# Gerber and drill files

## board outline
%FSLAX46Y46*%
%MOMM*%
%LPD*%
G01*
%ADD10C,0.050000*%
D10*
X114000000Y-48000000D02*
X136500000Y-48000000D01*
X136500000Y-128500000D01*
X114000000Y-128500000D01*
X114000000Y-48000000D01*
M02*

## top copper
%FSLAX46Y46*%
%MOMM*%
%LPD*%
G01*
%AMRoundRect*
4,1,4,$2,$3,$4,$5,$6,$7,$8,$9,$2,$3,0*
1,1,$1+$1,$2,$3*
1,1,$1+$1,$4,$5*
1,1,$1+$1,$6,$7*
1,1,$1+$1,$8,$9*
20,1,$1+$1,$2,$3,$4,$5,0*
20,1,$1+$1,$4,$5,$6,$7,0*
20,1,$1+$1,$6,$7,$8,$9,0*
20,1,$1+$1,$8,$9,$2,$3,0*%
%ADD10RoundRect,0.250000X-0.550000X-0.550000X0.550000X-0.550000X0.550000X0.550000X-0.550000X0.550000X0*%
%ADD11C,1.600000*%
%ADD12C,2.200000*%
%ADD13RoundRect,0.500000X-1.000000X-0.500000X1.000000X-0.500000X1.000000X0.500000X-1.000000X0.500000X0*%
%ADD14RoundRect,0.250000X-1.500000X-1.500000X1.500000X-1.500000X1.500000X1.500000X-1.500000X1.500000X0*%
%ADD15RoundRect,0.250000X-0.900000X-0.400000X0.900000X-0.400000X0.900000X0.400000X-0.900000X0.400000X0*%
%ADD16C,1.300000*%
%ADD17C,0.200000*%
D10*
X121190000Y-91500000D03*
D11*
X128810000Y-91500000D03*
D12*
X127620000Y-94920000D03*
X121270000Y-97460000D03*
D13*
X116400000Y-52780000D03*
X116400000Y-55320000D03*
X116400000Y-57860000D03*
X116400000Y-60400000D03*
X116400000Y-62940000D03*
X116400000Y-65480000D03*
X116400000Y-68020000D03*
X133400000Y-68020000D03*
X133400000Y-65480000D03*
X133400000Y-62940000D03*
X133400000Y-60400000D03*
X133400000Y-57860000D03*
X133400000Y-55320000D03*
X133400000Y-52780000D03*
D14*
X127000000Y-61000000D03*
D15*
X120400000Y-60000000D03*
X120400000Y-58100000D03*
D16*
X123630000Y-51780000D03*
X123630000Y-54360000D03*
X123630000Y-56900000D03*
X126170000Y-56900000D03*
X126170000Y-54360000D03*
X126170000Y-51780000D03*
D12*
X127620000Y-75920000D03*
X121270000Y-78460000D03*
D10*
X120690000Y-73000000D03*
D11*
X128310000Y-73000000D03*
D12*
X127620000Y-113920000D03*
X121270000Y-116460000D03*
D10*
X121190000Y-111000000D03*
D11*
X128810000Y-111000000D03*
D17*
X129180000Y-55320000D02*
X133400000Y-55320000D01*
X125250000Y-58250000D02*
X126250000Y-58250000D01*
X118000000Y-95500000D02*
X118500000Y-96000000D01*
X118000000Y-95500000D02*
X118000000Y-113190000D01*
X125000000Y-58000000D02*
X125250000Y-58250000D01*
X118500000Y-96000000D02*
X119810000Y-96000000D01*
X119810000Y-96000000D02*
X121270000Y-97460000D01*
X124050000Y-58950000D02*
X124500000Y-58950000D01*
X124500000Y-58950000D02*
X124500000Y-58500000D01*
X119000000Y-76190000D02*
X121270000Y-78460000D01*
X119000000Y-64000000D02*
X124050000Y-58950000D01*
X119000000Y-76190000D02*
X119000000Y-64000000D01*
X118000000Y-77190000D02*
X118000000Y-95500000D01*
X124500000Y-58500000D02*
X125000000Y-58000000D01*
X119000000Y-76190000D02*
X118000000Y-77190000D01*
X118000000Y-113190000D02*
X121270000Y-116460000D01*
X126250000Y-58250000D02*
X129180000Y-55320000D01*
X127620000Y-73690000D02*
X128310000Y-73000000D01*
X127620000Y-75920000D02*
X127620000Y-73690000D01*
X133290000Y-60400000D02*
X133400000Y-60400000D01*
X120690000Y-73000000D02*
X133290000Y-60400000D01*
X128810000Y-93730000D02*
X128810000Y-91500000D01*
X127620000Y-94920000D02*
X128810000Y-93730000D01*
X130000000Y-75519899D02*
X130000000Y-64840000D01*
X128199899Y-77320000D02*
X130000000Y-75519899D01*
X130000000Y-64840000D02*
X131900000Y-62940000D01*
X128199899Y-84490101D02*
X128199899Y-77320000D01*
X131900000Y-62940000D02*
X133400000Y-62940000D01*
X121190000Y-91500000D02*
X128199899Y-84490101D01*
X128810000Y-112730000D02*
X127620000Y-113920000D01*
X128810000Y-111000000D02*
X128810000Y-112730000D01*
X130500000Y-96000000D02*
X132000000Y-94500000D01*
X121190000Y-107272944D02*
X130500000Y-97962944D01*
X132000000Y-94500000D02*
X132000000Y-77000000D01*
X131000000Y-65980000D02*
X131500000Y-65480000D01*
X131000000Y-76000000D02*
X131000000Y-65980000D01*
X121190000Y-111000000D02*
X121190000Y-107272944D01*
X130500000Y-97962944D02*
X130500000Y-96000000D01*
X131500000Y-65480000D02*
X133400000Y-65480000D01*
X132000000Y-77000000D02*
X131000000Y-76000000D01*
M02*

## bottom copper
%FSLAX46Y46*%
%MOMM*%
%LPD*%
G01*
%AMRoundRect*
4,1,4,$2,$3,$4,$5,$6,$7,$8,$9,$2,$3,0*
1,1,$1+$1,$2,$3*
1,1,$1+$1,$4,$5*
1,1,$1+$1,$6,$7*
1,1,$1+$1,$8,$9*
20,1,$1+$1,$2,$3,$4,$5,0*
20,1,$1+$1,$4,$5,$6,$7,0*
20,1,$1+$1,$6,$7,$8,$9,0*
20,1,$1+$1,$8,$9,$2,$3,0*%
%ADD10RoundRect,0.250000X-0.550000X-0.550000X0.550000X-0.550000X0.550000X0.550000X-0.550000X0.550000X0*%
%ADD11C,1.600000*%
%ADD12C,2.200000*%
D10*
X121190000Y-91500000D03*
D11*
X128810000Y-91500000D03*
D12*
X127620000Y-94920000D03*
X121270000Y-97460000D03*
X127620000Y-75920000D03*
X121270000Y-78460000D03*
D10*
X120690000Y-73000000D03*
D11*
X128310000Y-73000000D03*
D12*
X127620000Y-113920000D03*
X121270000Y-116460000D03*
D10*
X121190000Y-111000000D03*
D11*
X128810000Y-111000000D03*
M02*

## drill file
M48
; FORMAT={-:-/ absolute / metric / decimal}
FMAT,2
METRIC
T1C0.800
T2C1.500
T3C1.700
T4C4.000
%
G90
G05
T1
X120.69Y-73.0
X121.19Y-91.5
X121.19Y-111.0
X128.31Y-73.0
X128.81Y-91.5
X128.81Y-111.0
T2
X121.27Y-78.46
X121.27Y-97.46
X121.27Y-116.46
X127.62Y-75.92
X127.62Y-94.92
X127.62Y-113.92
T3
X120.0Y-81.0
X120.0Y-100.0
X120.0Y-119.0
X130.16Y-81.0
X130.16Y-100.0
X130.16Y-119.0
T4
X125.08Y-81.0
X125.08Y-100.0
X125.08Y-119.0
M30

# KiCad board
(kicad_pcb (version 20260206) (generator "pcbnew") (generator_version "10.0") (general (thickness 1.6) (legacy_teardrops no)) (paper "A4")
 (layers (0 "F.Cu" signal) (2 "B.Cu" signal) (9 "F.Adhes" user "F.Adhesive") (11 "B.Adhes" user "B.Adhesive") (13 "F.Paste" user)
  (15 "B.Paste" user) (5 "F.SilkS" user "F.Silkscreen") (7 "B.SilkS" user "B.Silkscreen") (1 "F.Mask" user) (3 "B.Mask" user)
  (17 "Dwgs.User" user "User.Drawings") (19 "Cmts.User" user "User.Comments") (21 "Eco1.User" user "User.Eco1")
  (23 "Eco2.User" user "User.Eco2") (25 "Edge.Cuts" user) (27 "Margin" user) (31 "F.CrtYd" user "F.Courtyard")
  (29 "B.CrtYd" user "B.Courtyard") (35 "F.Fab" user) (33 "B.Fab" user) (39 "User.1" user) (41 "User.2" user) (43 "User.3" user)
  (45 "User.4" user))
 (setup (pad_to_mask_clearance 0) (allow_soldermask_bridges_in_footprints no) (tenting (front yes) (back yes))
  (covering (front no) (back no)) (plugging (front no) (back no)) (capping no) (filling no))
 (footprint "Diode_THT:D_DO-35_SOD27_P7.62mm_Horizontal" (layer "F.Cu") (at 121.19 91.5)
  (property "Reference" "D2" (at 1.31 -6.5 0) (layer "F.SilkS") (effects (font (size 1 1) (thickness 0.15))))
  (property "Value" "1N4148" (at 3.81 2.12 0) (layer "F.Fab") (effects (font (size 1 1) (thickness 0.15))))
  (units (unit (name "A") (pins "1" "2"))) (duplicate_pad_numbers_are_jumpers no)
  (pad "1" thru_hole roundrect (at 0 0) (size 1.6 1.6) (drill 0.8) (layers "*.Cu" "*.Mask") (remove_unused_layers no)
   (roundrect_rratio 0.15625) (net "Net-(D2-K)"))
  (pad "2" thru_hole circle (at 7.62 0) (size 1.6 1.6) (drill 0.8) (layers "*.Cu" "*.Mask") (remove_unused_layers no) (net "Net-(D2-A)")))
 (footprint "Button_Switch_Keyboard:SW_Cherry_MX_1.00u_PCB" (layer "F.Cu") (at 127.62 94.92)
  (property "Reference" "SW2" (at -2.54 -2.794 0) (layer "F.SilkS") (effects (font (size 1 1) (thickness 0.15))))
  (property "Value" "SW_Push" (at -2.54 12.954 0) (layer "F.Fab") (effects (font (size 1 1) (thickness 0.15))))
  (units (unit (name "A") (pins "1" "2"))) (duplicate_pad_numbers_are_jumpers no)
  (pad "" np_thru_hole circle (at -7.62 5.08) (size 1.7 1.7) (drill 1.7) (layers "*.Cu" "*.Mask"))
  (pad "" np_thru_hole circle (at -2.54 5.08) (size 4 4) (drill 4) (layers "*.Cu" "*.Mask"))
  (pad "" np_thru_hole circle (at 2.54 5.08) (size 1.7 1.7) (drill 1.7) (layers "*.Cu" "*.Mask"))
  (pad "1" thru_hole circle (at 0 0) (size 2.2 2.2) (drill 1.5) (layers "*.Cu" "*.Mask") (remove_unused_layers no) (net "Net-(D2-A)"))
  (pad "2" thru_hole circle (at -6.35 2.54) (size 2.2 2.2) (drill 1.5) (layers "*.Cu" "*.Mask") (remove_unused_layers no) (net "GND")))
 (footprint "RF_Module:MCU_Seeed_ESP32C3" (layer "F.Cu") (at 124.9 60.4)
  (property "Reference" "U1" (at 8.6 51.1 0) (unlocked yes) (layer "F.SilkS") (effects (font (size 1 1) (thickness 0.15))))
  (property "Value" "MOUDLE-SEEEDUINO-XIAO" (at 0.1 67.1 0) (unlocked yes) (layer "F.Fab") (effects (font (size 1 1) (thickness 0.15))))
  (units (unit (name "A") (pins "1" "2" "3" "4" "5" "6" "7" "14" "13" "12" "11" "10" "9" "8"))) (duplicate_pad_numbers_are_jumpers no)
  (pad "" smd roundrect (at 1.1 -0.4) (size 1.5 1.5) (layers "F.Paste") (roundrect_rratio 0.1666666667))
  (pad "" smd roundrect (at 1.1 1.6) (size 1.5 1.5) (layers "F.Paste") (roundrect_rratio 0.1666666667))
  (pad "" smd roundrect (at 3.1 -0.4) (size 1.5 1.5) (layers "F.Paste") (roundrect_rratio 0.1666666667))
  (pad "" smd roundrect (at 3.1 1.6) (size 1.5 1.5) (layers "F.Paste") (roundrect_rratio 0.1666666667))
  (pad "1" smd roundrect (at -8.5 -7.62) (size 3 2) (layers "F.Cu" "F.Mask" "F.Paste") (roundrect_rratio 0.25)
   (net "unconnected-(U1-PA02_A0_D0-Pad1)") (thermal_bridge_angle 45))
  (pad "2" smd roundrect (at -8.5 -5.08) (size 3 2) (layers "F.Cu" "F.Mask" "F.Paste") (roundrect_rratio 0.25)
   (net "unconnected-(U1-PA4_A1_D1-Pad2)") (thermal_bridge_angle 45))
  (pad "3" smd roundrect (at -8.5 -2.54) (size 3 2) (layers "F.Cu" "F.Mask" "F.Paste") (roundrect_rratio 0.25)
   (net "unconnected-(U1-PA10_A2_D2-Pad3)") (thermal_bridge_angle 45))
  (pad "4" smd roundrect (at -8.5 0) (size 3 2) (layers "F.Cu" "F.Mask" "F.Paste") (roundrect_rratio 0.25)
   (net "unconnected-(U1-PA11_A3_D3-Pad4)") (thermal_bridge_angle 45))
  (pad "5" smd roundrect (at -8.5 2.54) (size 3 2) (layers "F.Cu" "F.Mask" "F.Paste") (roundrect_rratio 0.25)
   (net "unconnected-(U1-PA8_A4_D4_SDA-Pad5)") (thermal_bridge_angle 45))
  (pad "6" smd roundrect (at -8.5 5.08) (size 3 2) (layers "F.Cu" "F.Mask" "F.Paste") (roundrect_rratio 0.25)
   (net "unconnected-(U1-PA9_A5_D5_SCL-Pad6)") (thermal_bridge_angle 45))
  (pad "7" smd roundrect (at -8.5 7.62) (size 3 2) (layers "F.Cu" "F.Mask" "F.Paste") (roundrect_rratio 0.25)
   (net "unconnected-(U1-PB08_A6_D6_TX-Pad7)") (thermal_bridge_angle 45))
  (pad "8" smd roundrect (at 8.5 7.62) (size 3 2) (layers "F.Cu" "F.Mask" "F.Paste") (roundrect_rratio 0.25)
   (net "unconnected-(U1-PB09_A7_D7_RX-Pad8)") (thermal_bridge_angle 45))
  (pad "9" smd roundrect (at 8.5 5.08) (size 3 2) (layers "F.Cu" "F.Mask" "F.Paste") (roundrect_rratio 0.25) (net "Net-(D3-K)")
   (thermal_bridge_angle 45))
  (pad "10" smd roundrect (at 8.5 2.54) (size 3 2) (layers "F.Cu" "F.Mask" "F.Paste") (roundrect_rratio 0.25) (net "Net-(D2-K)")
   (thermal_bridge_angle 45))
  (pad "11" smd roundrect (at 8.5 0) (size 3 2) (layers "F.Cu" "F.Mask" "F.Paste") (roundrect_rratio 0.25) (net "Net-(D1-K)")
   (thermal_bridge_angle 45))
  (pad "12" smd roundrect (at 8.5 -2.54) (size 3 2) (layers "F.Cu" "F.Mask" "F.Paste") (roundrect_rratio 0.25)
   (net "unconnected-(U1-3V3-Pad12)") (thermal_bridge_angle 45))
  (pad "13" smd roundrect (at 8.5 -5.08) (size 3 2) (layers "F.Cu" "F.Mask" "F.Paste") (roundrect_rratio 0.25) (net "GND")
   (thermal_bridge_angle 45))
  (pad "14" smd roundrect (at 8.5 -7.62) (size 3 2) (layers "F.Cu" "F.Mask" "F.Paste") (roundrect_rratio 0.25)
   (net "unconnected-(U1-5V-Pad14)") (thermal_bridge_angle 45))
  (pad "15" smd roundrect (at 2.1 0.6) (size 3.5 3.5) (layers "F.Cu" "F.Mask") (roundrect_rratio 0.07142857143))
  (pad "16" smd roundrect (at -4.5 -0.4) (size 2.3 1.3) (layers "F.Cu" "F.Mask" "F.Paste") (roundrect_rratio 0.1923076923))
  (pad "17" smd roundrect (at -4.5 -2.3) (size 2.3 1.3) (layers "F.Cu" "F.Mask" "F.Paste") (roundrect_rratio 0.1923076923))
  (pad "18" smd circle (at -1.27 -8.62) (size 1.3 1.3) (layers "F.Cu" "F.Mask" "F.Paste"))
  (pad "19" smd circle (at -1.27 -6.04) (size 1.3 1.3) (layers "F.Cu" "F.Mask" "F.Paste"))
  (pad "20" smd circle (at -1.27 -3.5) (size 1.3 1.3) (layers "F.Cu" "F.Mask" "F.Paste"))
  (pad "21" smd circle (at 1.27 -3.5) (size 1.3 1.3) (layers "F.Cu" "F.Mask" "F.Paste"))
  (pad "22" smd circle (at 1.27 -6.04) (size 1.3 1.3) (layers "F.Cu" "F.Mask" "F.Paste"))
  (pad "23" smd circle (at 1.27 -8.62) (size 1.3 1.3) (layers "F.Cu" "F.Mask" "F.Paste")))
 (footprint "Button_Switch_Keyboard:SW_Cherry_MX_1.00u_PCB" (layer "F.Cu") (at 127.62 75.92)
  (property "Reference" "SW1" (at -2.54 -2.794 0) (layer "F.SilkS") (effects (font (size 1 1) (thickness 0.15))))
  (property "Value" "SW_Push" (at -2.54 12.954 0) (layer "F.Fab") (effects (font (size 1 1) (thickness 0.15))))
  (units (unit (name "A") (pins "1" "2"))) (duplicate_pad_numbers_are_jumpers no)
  (pad "" np_thru_hole circle (at -7.62 5.08) (size 1.7 1.7) (drill 1.7) (layers "*.Cu" "*.Mask"))
  (pad "" np_thru_hole circle (at -2.54 5.08) (size 4 4) (drill 4) (layers "*.Cu" "*.Mask"))
  (pad "" np_thru_hole circle (at 2.54 5.08) (size 1.7 1.7) (drill 1.7) (layers "*.Cu" "*.Mask"))
  (pad "1" thru_hole circle (at 0 0) (size 2.2 2.2) (drill 1.5) (layers "*.Cu" "*.Mask") (remove_unused_layers no) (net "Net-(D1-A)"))
  (pad "2" thru_hole circle (at -6.35 2.54) (size 2.2 2.2) (drill 1.5) (layers "*.Cu" "*.Mask") (remove_unused_layers no) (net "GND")))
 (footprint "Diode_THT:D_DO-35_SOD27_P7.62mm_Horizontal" (layer "F.Cu") (at 120.69 73)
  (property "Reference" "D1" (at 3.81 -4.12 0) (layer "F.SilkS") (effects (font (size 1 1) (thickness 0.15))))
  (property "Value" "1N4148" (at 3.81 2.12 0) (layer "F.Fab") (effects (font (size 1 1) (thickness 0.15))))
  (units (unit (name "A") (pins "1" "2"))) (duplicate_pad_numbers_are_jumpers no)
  (pad "1" thru_hole roundrect (at 0 0) (size 1.6 1.6) (drill 0.8) (layers "*.Cu" "*.Mask") (remove_unused_layers no)
   (roundrect_rratio 0.15625) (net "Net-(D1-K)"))
  (pad "2" thru_hole circle (at 7.62 0) (size 1.6 1.6) (drill 0.8) (layers "*.Cu" "*.Mask") (remove_unused_layers no) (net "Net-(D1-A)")))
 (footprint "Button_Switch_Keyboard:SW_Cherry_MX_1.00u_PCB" (layer "F.Cu") (at 127.62 113.92)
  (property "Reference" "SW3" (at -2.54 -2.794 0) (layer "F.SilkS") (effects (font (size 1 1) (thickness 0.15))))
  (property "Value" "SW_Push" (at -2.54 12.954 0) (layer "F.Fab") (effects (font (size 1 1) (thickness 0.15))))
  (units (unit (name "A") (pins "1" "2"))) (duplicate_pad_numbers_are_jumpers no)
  (pad "" np_thru_hole circle (at -7.62 5.08) (size 1.7 1.7) (drill 1.7) (layers "*.Cu" "*.Mask"))
  (pad "" np_thru_hole circle (at -2.54 5.08) (size 4 4) (drill 4) (layers "*.Cu" "*.Mask"))
  (pad "" np_thru_hole circle (at 2.54 5.08) (size 1.7 1.7) (drill 1.7) (layers "*.Cu" "*.Mask"))
  (pad "1" thru_hole circle (at 0 0) (size 2.2 2.2) (drill 1.5) (layers "*.Cu" "*.Mask") (remove_unused_layers no) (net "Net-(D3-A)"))
  (pad "2" thru_hole circle (at -6.35 2.54) (size 2.2 2.2) (drill 1.5) (layers "*.Cu" "*.Mask") (remove_unused_layers no) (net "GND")))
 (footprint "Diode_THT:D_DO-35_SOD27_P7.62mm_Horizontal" (layer "F.Cu") (at 121.19 111)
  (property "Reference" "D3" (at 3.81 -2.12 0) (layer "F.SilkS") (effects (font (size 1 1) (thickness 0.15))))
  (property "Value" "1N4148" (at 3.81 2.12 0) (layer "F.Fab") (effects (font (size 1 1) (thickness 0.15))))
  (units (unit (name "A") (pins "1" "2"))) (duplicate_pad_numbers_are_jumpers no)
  (pad "1" thru_hole roundrect (at 0 0) (size 1.6 1.6) (drill 0.8) (layers "*.Cu" "*.Mask") (remove_unused_layers no)
   (roundrect_rratio 0.15625) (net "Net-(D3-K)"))
  (pad "2" thru_hole circle (at 7.62 0) (size 1.6 1.6) (drill 0.8) (layers "*.Cu" "*.Mask") (remove_unused_layers no) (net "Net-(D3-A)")))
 (gr_rect (start 114 48) (end 136.5 128.5) (stroke (width 0.05) (type default)) (fill no) (layer "Edge.Cuts"))
 (segment (start 129.18 55.32) (end 133.4 55.32) (width 0.2) (layer "F.Cu") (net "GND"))
 (segment (start 125.25 58.25) (end 126.25 58.25) (width 0.2) (layer "F.Cu") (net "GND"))
 (segment (start 118 95.5) (end 118.5 96) (width 0.2) (layer "F.Cu") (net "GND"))
 (segment (start 118 95.5) (end 118 113.19) (width 0.2) (layer "F.Cu") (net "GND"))
 (segment (start 125 58) (end 125.25 58.25) (width 0.2) (layer "F.Cu") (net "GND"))
 (segment (start 118.5 96) (end 119.81 96) (width 0.2) (layer "F.Cu") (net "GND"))
 (segment (start 119.81 96) (end 121.27 97.46) (width 0.2) (layer "F.Cu") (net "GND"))
 (segment (start 124.05 58.95) (end 124.5 58.95) (width 0.2) (layer "F.Cu") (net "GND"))
 (segment (start 124.5 58.95) (end 124.5 58.5) (width 0.2) (layer "F.Cu") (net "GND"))
 (segment (start 119 76.19) (end 121.27 78.46) (width 0.2) (layer "F.Cu") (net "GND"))
 (segment (start 119 64) (end 124.05 58.95) (width 0.2) (layer "F.Cu") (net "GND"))
 (segment (start 119 76.19) (end 119 64) (width 0.2) (layer "F.Cu") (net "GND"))
 (segment (start 118 77.19) (end 118 95.5) (width 0.2) (layer "F.Cu") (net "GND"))
 (segment (start 124.5 58.5) (end 125 58) (width 0.2) (layer "F.Cu") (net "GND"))
 (segment (start 119 76.19) (end 118 77.19) (width 0.2) (layer "F.Cu") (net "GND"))
 (segment (start 118 113.19) (end 121.27 116.46) (width 0.2) (layer "F.Cu") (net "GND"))
 (segment (start 126.25 58.25) (end 129.18 55.32) (width 0.2) (layer "F.Cu") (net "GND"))
 (segment (start 127.62 73.69) (end 128.31 73) (width 0.2) (layer "F.Cu") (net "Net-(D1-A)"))
 (segment (start 127.62 75.92) (end 127.62 73.69) (width 0.2) (layer "F.Cu") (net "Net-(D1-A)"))
 (segment (start 133.29 60.4) (end 133.4 60.4) (width 0.2) (layer "F.Cu") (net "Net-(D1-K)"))
 (segment (start 120.69 73) (end 133.29 60.4) (width 0.2) (layer "F.Cu") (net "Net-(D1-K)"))
 (segment (start 128.81 93.73) (end 128.81 91.5) (width 0.2) (layer "F.Cu") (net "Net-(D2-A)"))
 (segment (start 127.62 94.92) (end 128.81 93.73) (width 0.2) (layer "F.Cu") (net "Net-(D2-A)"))
 (segment (start 130 75.519899) (end 130 64.84) (width 0.2) (layer "F.Cu") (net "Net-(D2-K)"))
 (segment (start 128.199899 77.32) (end 130 75.519899) (width 0.2) (layer "F.Cu") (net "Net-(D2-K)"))
 (segment (start 130 64.84) (end 131.9 62.94) (width 0.2) (layer "F.Cu") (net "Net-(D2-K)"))
 (segment (start 128.199899 84.490101) (end 128.199899 77.32) (width 0.2) (layer "F.Cu") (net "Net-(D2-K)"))
 (segment (start 131.9 62.94) (end 133.4 62.94) (width 0.2) (layer "F.Cu") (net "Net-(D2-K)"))
 (segment (start 121.19 91.5) (end 128.199899 84.490101) (width 0.2) (layer "F.Cu") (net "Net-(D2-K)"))
 (segment (start 128.81 112.73) (end 127.62 113.92) (width 0.2) (layer "F.Cu") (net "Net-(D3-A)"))
 (segment (start 128.81 111) (end 128.81 112.73) (width 0.2) (layer "F.Cu") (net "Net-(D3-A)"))
 (segment (start 130.5 96) (end 132 94.5) (width 0.2) (layer "F.Cu") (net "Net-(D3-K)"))
 (segment (start 121.19 107.272944) (end 130.5 97.962944) (width 0.2) (layer "F.Cu") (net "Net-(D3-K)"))
 (segment (start 132 94.5) (end 132 77) (width 0.2) (layer "F.Cu") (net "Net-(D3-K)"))
 (segment (start 131 65.98) (end 131.5 65.48) (width 0.2) (layer "F.Cu") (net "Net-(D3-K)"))
 (segment (start 131 76) (end 131 65.98) (width 0.2) (layer "F.Cu") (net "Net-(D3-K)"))
 (segment (start 121.19 111) (end 121.19 107.272944) (width 0.2) (layer "F.Cu") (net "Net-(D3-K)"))
 (segment (start 130.5 97.962944) (end 130.5 96) (width 0.2) (layer "F.Cu") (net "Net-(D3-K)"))
 (segment (start 131.5 65.48) (end 133.4 65.48) (width 0.2) (layer "F.Cu") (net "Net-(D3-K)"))
 (segment (start 132 77) (end 131 76) (width 0.2) (layer "F.Cu") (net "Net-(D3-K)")))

